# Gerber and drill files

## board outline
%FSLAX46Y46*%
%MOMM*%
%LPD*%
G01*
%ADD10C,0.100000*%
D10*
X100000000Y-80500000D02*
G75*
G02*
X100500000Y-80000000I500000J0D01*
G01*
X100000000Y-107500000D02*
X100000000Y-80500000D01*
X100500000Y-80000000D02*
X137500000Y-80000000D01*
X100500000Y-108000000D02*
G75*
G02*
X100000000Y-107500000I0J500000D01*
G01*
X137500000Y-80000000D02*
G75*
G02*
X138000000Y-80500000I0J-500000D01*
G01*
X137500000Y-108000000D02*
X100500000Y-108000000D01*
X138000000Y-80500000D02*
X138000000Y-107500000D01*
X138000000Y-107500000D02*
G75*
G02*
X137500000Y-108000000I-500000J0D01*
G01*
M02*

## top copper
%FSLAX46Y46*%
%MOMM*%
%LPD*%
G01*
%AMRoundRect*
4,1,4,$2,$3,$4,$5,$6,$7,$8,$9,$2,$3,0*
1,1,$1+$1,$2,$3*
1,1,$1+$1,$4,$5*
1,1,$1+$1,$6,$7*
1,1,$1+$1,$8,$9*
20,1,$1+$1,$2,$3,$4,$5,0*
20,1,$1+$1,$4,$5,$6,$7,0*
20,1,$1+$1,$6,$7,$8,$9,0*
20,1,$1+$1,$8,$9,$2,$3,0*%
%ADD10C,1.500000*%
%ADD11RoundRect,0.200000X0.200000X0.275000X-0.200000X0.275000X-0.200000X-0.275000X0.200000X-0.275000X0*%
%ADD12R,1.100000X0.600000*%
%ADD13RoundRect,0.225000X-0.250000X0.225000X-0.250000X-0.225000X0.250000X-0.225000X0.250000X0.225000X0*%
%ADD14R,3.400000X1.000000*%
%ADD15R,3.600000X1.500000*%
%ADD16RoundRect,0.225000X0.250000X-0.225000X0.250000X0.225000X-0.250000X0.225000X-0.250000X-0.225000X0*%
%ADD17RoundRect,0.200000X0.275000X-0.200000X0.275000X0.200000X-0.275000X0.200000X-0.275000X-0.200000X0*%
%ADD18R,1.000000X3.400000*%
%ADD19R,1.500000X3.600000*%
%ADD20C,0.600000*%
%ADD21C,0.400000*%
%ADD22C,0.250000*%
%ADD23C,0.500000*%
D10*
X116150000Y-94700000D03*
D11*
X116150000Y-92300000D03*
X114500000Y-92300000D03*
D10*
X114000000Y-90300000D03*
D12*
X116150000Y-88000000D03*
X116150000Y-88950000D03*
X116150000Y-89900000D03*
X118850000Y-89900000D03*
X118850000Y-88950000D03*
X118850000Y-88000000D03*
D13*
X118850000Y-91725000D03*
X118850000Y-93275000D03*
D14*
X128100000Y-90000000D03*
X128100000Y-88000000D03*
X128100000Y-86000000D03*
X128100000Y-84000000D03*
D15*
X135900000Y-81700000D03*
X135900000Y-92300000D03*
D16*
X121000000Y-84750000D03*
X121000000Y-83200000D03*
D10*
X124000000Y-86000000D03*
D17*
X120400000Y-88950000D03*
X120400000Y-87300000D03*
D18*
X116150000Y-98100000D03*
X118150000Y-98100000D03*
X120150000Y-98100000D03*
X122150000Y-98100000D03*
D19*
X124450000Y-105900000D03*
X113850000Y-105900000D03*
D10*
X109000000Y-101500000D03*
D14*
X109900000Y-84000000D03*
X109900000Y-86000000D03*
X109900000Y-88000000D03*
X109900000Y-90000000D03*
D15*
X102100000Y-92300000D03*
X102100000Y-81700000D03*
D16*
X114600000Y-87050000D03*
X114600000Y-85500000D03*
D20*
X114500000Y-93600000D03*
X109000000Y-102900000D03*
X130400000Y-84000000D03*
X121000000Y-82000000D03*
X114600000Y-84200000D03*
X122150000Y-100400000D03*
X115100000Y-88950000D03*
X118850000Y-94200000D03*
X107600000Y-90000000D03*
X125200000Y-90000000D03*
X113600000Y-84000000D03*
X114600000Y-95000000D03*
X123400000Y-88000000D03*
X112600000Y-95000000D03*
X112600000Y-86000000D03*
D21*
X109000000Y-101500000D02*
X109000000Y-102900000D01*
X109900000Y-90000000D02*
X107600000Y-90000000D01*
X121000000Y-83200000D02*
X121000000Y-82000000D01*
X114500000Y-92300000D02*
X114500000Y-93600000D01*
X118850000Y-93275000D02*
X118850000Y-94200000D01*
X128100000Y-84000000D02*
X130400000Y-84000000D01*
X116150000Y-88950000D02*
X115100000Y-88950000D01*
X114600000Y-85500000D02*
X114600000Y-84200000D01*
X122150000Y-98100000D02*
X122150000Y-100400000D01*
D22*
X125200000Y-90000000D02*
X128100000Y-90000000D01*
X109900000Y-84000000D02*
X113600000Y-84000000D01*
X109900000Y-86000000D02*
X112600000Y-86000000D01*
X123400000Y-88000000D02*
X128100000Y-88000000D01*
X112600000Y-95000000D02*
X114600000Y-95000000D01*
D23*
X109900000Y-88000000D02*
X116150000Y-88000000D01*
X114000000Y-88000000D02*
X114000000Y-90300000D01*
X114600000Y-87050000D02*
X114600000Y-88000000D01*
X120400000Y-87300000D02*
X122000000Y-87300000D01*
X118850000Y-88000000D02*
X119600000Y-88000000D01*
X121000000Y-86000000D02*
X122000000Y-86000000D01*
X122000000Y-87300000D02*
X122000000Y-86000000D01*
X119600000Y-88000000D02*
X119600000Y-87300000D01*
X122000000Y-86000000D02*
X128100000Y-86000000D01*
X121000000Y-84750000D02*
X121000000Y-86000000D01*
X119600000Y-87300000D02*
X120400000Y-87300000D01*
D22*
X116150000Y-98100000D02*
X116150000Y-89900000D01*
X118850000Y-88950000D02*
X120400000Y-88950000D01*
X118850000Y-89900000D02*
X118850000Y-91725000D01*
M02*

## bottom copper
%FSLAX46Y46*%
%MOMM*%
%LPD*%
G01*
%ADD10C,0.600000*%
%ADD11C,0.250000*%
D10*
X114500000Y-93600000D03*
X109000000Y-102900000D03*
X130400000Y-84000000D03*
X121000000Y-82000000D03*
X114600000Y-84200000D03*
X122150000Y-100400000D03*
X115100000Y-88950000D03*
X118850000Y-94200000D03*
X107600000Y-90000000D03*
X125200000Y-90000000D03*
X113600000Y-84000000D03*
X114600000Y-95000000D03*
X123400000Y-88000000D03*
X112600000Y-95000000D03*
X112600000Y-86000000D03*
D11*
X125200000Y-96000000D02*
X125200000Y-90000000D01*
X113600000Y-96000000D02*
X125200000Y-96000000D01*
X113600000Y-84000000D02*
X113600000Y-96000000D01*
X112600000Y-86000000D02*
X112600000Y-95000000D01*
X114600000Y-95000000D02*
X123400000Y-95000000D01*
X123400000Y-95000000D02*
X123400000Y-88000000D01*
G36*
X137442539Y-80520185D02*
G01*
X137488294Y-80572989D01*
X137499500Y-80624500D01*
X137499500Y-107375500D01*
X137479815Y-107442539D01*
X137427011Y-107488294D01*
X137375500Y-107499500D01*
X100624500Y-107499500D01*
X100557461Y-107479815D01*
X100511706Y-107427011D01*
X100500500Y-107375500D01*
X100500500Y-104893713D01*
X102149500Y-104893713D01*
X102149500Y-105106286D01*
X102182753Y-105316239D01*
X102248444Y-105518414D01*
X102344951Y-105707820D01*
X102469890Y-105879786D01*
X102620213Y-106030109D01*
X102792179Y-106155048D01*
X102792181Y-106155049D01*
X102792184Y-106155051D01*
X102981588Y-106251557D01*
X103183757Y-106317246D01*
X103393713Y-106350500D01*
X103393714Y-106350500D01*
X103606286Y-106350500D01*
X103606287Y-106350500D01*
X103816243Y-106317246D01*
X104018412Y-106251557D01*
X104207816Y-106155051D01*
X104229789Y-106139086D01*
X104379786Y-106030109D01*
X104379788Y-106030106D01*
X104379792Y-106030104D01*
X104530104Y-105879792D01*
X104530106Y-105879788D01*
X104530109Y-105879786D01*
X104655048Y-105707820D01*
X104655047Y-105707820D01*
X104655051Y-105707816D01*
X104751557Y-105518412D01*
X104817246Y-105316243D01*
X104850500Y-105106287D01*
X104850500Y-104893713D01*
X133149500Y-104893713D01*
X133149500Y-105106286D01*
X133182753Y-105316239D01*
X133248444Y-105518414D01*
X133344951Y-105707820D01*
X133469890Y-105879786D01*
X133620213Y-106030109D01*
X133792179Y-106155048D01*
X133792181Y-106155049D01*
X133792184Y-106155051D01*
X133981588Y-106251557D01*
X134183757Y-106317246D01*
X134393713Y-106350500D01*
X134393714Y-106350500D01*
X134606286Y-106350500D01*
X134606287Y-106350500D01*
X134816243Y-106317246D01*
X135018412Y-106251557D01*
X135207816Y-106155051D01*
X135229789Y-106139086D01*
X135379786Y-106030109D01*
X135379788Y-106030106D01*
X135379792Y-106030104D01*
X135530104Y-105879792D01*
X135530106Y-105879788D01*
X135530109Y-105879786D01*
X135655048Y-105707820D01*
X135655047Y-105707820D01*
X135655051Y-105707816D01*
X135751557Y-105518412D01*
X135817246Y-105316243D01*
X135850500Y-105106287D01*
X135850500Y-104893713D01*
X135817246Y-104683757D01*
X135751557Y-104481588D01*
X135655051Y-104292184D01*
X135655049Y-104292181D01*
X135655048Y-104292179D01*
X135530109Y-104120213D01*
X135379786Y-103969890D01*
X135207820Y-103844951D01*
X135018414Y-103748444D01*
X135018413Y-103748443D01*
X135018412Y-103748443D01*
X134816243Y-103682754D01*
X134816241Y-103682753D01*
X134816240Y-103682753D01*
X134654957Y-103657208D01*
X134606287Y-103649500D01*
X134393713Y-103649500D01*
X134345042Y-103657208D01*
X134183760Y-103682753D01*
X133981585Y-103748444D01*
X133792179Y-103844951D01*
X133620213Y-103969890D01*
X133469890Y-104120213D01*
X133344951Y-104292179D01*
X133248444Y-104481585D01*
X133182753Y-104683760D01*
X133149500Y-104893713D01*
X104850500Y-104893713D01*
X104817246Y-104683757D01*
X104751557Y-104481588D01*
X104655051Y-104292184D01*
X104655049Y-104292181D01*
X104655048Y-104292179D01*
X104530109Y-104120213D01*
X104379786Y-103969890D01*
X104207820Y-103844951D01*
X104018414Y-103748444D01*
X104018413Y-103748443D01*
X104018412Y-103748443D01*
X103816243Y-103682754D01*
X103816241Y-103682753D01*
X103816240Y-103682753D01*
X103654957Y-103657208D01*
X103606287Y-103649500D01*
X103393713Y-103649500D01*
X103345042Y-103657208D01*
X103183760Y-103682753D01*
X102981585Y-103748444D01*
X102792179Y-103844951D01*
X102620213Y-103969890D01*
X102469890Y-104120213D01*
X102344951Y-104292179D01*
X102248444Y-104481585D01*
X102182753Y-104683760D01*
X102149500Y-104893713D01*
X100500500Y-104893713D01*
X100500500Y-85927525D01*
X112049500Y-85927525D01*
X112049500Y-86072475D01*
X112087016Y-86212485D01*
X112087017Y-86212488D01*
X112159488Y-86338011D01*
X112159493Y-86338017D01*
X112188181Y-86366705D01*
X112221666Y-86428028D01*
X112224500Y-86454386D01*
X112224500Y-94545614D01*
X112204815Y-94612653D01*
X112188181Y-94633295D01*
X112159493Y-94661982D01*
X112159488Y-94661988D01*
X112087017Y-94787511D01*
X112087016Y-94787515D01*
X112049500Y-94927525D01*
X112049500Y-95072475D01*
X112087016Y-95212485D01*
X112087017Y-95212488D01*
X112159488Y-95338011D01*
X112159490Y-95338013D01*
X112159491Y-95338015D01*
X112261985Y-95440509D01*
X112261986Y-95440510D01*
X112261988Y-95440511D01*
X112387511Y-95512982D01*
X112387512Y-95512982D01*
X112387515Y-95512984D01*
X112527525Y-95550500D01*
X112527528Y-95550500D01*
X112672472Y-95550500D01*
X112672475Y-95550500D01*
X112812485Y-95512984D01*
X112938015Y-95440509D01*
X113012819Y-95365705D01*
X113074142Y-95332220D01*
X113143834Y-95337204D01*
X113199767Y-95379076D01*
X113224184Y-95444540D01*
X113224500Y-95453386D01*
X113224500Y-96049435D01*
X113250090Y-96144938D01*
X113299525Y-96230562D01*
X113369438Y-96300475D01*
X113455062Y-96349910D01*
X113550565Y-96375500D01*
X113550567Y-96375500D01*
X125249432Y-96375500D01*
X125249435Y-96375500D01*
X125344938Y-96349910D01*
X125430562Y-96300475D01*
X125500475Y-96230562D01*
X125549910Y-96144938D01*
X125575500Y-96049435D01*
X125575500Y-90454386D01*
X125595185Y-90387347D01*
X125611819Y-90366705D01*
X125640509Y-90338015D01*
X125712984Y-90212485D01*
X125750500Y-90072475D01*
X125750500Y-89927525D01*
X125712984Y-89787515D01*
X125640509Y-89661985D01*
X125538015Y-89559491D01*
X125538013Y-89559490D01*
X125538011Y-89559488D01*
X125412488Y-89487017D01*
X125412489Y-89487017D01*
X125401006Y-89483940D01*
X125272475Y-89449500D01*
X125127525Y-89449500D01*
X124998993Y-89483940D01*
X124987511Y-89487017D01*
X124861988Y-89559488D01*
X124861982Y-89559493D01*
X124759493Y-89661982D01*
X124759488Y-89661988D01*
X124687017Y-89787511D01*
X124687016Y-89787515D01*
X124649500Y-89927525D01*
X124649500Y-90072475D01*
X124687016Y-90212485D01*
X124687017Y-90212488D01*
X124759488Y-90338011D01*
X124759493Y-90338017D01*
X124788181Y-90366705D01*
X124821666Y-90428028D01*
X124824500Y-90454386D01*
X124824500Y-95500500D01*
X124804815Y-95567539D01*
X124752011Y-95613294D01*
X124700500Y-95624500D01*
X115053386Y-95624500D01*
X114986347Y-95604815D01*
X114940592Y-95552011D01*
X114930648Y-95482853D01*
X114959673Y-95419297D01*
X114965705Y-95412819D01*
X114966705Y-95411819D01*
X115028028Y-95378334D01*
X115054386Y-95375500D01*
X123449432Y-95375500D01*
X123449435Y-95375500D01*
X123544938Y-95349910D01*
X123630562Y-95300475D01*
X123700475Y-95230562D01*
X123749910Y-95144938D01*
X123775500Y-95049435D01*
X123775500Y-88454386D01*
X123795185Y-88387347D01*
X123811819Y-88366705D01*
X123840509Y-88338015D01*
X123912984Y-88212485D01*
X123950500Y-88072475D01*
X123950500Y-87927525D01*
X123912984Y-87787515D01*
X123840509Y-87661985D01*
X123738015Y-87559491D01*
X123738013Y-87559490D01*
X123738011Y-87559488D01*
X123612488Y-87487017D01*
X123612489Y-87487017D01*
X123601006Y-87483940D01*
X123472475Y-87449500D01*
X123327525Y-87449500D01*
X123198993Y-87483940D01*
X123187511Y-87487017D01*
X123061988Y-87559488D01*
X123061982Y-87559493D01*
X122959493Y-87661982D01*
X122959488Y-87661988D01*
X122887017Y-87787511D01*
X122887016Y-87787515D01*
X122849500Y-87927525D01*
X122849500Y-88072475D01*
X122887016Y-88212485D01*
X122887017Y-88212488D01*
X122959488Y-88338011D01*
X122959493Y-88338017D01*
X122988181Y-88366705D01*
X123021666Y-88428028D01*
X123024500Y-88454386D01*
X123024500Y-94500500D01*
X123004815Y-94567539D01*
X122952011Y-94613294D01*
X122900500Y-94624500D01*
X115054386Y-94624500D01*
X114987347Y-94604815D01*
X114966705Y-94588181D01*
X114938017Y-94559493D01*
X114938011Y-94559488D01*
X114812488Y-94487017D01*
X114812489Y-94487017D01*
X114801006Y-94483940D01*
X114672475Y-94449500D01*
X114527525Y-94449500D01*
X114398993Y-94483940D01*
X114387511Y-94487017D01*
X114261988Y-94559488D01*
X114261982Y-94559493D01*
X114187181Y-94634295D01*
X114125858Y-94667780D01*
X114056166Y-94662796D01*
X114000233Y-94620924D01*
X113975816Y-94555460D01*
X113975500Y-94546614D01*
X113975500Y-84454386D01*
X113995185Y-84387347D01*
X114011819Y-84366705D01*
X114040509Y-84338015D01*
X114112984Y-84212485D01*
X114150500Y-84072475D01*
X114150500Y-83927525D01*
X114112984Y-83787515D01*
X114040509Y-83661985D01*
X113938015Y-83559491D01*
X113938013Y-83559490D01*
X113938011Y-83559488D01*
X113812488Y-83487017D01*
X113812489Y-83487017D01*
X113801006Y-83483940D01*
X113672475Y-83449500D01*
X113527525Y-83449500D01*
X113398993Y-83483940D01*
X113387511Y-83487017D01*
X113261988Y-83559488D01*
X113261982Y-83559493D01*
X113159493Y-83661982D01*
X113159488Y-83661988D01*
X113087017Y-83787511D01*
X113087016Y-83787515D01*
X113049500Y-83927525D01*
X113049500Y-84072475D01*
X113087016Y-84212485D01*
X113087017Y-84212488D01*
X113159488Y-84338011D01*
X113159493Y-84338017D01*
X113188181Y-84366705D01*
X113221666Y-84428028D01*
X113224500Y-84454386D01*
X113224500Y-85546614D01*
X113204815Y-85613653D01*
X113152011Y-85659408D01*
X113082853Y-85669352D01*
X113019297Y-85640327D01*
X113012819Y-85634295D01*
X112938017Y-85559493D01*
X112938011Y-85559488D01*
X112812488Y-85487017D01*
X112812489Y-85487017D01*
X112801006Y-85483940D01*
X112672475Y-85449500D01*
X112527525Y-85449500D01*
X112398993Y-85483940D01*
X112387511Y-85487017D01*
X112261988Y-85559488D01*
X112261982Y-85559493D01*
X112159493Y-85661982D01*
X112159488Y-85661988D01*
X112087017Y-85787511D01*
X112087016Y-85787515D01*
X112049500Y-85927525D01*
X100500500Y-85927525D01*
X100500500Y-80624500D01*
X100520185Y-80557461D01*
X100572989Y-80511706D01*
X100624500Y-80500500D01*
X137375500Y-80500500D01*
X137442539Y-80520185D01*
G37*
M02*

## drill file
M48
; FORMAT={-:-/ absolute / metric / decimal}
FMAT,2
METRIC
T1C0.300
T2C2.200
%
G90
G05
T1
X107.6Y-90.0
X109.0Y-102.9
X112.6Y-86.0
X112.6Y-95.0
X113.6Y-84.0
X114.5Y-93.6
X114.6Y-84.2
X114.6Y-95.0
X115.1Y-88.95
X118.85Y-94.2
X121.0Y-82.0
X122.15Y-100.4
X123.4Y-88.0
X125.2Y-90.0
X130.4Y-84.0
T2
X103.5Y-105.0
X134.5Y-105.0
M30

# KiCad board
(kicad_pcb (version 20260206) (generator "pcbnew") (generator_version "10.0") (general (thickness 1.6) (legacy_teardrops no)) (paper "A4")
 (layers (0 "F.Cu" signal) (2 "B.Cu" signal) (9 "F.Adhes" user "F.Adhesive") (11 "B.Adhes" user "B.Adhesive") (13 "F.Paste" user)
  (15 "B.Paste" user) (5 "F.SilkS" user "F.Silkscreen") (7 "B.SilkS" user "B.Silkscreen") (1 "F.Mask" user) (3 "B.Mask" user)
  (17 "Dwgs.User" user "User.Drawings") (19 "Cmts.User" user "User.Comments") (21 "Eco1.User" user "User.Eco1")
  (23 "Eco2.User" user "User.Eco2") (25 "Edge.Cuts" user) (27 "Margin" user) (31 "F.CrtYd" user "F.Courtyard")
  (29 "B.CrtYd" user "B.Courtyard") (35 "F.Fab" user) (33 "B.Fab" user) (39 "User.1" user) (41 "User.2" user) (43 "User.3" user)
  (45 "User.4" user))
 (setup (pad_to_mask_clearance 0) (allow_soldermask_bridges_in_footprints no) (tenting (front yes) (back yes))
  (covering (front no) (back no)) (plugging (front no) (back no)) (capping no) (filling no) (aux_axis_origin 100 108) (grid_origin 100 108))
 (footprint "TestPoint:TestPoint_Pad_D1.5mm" (layer "F.Cu") (at 116.15 94.7)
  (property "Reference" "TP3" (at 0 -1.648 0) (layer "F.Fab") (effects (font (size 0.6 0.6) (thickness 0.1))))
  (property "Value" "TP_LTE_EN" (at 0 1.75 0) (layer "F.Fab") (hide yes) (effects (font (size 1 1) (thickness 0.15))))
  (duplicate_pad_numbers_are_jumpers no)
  (pad "1" smd circle (at 0 0) (size 1.5 1.5) (layers "F.Cu" "F.Mask") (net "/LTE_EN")))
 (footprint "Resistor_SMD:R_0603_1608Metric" (layer "F.Cu") (at 115.325 92.3 180)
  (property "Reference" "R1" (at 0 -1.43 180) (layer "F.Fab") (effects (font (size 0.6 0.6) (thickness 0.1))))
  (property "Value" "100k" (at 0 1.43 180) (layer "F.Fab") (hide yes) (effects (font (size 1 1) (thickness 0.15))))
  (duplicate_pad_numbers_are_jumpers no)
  (pad "1" smd roundrect (at -0.825 0 180) (size 0.8 0.95) (layers "F.Cu" "F.Mask" "F.Paste") (roundrect_rratio 0.25) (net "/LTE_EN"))
  (pad "2" smd roundrect (at 0.825 0 180) (size 0.8 0.95) (layers "F.Cu" "F.Mask" "F.Paste") (roundrect_rratio 0.25) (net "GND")))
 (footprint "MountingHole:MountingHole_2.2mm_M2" (layer "F.Cu") (at 134.5 105)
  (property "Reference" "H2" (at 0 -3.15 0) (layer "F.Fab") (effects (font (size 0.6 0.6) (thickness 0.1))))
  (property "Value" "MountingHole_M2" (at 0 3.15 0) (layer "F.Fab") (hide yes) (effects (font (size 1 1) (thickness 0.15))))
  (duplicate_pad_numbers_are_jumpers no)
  (pad "" np_thru_hole circle (at 0 0) (size 2.2 2.2) (drill 2.2) (layers "*.Cu" "*.Mask")))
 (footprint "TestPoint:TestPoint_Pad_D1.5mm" (layer "F.Cu") (at 114 90.3)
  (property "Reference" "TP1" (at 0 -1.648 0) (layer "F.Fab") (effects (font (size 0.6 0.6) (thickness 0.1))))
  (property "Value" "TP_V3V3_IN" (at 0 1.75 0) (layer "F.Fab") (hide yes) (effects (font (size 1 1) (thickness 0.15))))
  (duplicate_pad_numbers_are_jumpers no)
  (pad "1" smd circle (at 0 0) (size 1.5 1.5) (layers "F.Cu" "F.Mask") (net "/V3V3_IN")))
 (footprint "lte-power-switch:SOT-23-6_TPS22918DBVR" (layer "F.Cu") (at 117.5 88.95 180)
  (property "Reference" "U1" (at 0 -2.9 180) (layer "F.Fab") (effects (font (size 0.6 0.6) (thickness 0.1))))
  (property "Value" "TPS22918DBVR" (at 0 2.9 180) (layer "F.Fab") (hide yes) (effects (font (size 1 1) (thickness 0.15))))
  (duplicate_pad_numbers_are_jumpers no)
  (pad "1" smd rect (at 1.35 0.95 180) (size 1.1 0.6) (layers "F.Cu" "F.Mask" "F.Paste") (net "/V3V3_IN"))
  (pad "2" smd rect (at 1.35 0 180) (size 1.1 0.6) (layers "F.Cu" "F.Mask" "F.Paste") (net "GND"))
  (pad "3" smd rect (at 1.35 -0.95 180) (size 1.1 0.6) (layers "F.Cu" "F.Mask" "F.Paste") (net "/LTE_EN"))
  (pad "4" smd rect (at -1.35 -0.95 180) (size 1.1 0.6) (layers "F.Cu" "F.Mask" "F.Paste") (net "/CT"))
  (pad "5" smd rect (at -1.35 0 180) (size 1.1 0.6) (layers "F.Cu" "F.Mask" "F.Paste") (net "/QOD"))
  (pad "6" smd rect (at -1.35 0.95 180) (size 1.1 0.6) (layers "F.Cu" "F.Mask" "F.Paste") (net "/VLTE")))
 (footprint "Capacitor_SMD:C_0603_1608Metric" (layer "F.Cu") (at 118.85 92.5 -90)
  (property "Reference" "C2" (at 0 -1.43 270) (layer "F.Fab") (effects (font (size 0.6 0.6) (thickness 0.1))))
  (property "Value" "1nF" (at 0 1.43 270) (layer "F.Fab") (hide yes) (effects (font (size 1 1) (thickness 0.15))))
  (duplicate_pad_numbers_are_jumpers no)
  (pad "1" smd roundrect (at -0.775 0 270) (size 0.9 0.95) (layers "F.Cu" "F.Mask" "F.Paste") (roundrect_rratio 0.25) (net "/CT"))
  (pad "2" smd roundrect (at 0.775 0 270) (size 0.9 0.95) (layers "F.Cu" "F.Mask" "F.Paste") (roundrect_rratio 0.25) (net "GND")))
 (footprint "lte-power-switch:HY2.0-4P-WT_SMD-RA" (layer "F.Cu") (at 132 87 90)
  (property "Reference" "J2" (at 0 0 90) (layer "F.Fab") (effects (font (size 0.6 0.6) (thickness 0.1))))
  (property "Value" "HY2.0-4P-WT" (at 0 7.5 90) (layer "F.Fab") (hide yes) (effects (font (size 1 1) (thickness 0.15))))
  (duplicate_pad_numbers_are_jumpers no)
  (pad "1" smd rect (at -3 -3.9 90) (size 1 3.4) (layers "F.Cu" "F.Mask" "F.Paste") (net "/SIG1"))
  (pad "2" smd rect (at -1 -3.9 90) (size 1 3.4) (layers "F.Cu" "F.Mask" "F.Paste") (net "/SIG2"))
  (pad "3" smd rect (at 1 -3.9 90) (size 1 3.4) (layers "F.Cu" "F.Mask" "F.Paste") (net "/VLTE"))
  (pad "4" smd rect (at 3 -3.9 90) (size 1 3.4) (layers "F.Cu" "F.Mask" "F.Paste") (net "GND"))
  (pad "5" smd rect (at 5.3 3.9 90) (size 1.5 3.6) (layers "F.Cu" "F.Mask" "F.Paste"))
  (pad "6" smd rect (at -5.3 3.9 90) (size 1.5 3.6) (layers "F.Cu" "F.Mask" "F.Paste")))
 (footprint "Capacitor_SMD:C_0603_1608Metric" (layer "F.Cu") (at 121 83.975 90)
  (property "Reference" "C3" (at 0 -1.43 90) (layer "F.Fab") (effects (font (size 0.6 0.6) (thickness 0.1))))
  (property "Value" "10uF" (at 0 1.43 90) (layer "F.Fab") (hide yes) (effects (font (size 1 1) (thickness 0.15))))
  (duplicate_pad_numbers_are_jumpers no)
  (pad "1" smd roundrect (at -0.775 0 90) (size 0.9 0.95) (layers "F.Cu" "F.Mask" "F.Paste") (roundrect_rratio 0.25) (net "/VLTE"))
  (pad "2" smd roundrect (at 0.775 0 90) (size 0.9 0.95) (layers "F.Cu" "F.Mask" "F.Paste") (roundrect_rratio 0.25) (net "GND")))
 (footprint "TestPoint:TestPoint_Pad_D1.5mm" (layer "F.Cu") (at 124 86)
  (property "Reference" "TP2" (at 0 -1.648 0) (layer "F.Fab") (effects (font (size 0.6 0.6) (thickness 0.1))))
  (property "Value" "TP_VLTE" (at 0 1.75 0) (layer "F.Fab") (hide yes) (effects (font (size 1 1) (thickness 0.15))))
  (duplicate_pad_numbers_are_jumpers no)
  (pad "1" smd circle (at 0 0) (size 1.5 1.5) (layers "F.Cu" "F.Mask") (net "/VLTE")))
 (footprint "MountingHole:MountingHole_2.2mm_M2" (layer "F.Cu") (at 103.5 105)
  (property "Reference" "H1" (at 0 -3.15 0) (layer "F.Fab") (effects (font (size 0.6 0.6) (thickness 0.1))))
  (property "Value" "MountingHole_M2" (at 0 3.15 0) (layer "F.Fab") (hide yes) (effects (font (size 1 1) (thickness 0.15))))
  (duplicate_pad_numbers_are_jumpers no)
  (pad "" np_thru_hole circle (at 0 0) (size 2.2 2.2) (drill 2.2) (layers "*.Cu" "*.Mask")))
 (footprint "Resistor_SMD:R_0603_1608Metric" (layer "F.Cu") (at 120.4 88.125 90)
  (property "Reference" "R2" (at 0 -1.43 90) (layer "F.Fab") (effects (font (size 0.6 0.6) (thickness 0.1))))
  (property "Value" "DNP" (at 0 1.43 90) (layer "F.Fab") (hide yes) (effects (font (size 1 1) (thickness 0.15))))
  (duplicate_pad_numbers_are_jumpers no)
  (pad "1" smd roundrect (at -0.825 0 90) (size 0.8 0.95) (layers "F.Cu" "F.Mask" "F.Paste") (roundrect_rratio 0.25) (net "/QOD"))
  (pad "2" smd roundrect (at 0.825 0 90) (size 0.8 0.95) (layers "F.Cu" "F.Mask" "F.Paste") (roundrect_rratio 0.25) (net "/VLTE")))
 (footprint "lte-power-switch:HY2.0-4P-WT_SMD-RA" (layer "F.Cu") (at 119.15 102)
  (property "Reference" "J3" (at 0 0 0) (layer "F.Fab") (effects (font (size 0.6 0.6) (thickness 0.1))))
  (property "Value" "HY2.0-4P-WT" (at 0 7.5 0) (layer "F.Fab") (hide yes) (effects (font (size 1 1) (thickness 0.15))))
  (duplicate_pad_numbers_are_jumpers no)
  (pad "1" smd rect (at -3 -3.9) (size 1 3.4) (layers "F.Cu" "F.Mask" "F.Paste") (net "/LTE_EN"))
  (pad "2" smd rect (at -1 -3.9) (size 1 3.4) (layers "F.Cu" "F.Mask" "F.Paste") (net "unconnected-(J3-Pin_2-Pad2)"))
  (pad "3" smd rect (at 1 -3.9) (size 1 3.4) (layers "F.Cu" "F.Mask" "F.Paste") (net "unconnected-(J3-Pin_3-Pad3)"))
  (pad "4" smd rect (at 3 -3.9) (size 1 3.4) (layers "F.Cu" "F.Mask" "F.Paste") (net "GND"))
  (pad "5" smd rect (at 5.3 3.9) (size 1.5 3.6) (layers "F.Cu" "F.Mask" "F.Paste"))
  (pad "6" smd rect (at -5.3 3.9) (size 1.5 3.6) (layers "F.Cu" "F.Mask" "F.Paste")))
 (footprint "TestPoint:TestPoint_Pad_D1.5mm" (layer "F.Cu") (at 109 101.5)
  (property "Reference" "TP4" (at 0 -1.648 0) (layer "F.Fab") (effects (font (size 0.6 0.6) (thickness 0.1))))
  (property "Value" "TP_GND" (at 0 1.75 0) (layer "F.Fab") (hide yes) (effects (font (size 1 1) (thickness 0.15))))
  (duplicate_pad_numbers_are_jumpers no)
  (pad "1" smd circle (at 0 0) (size 1.5 1.5) (layers "F.Cu" "F.Mask") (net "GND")))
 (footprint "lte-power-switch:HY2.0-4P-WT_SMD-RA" (layer "F.Cu") (at 106 87 -90)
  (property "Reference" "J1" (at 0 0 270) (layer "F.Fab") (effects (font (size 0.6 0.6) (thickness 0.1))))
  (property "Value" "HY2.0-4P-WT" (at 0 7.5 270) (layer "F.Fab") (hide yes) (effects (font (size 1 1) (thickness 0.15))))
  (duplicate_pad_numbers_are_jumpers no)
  (pad "1" smd rect (at -3 -3.9 270) (size 1 3.4) (layers "F.Cu" "F.Mask" "F.Paste") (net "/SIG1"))
  (pad "2" smd rect (at -1 -3.9 270) (size 1 3.4) (layers "F.Cu" "F.Mask" "F.Paste") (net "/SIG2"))
  (pad "3" smd rect (at 1 -3.9 270) (size 1 3.4) (layers "F.Cu" "F.Mask" "F.Paste") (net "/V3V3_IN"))
  (pad "4" smd rect (at 3 -3.9 270) (size 1 3.4) (layers "F.Cu" "F.Mask" "F.Paste") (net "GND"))
  (pad "5" smd rect (at 5.3 3.9 270) (size 1.5 3.6) (layers "F.Cu" "F.Mask" "F.Paste"))
  (pad "6" smd rect (at -5.3 3.9 270) (size 1.5 3.6) (layers "F.Cu" "F.Mask" "F.Paste")))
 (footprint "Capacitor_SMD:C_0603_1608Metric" (layer "F.Cu") (at 114.6 86.275 90)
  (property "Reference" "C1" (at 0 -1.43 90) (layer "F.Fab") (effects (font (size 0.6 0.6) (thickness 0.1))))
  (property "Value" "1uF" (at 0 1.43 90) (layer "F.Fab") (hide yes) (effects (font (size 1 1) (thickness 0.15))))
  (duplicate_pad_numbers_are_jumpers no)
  (pad "1" smd roundrect (at -0.775 0 90) (size 0.9 0.95) (layers "F.Cu" "F.Mask" "F.Paste") (roundrect_rratio 0.25) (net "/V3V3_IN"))
  (pad "2" smd roundrect (at 0.775 0 90) (size 0.9 0.95) (layers "F.Cu" "F.Mask" "F.Paste") (roundrect_rratio 0.25) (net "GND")))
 (gr_arc (start 100 80.5) (mid 100.146446 80.146446) (end 100.5 80) (stroke (width 0.1) (type default)) (layer "Edge.Cuts"))
 (gr_line (start 100 107.5) (end 100 80.5) (stroke (width 0.1) (type default)) (layer "Edge.Cuts"))
 (gr_line (start 100.5 80) (end 137.5 80) (stroke (width 0.1) (type default)) (layer "Edge.Cuts"))
 (gr_arc (start 100.5 108) (mid 100.146446 107.853553) (end 100 107.5) (stroke (width 0.1) (type default)) (layer "Edge.Cuts"))
 (gr_arc (start 137.5 80) (mid 137.853553 80.146446) (end 138 80.5) (stroke (width 0.1) (type default)) (layer "Edge.Cuts"))
 (gr_line (start 137.5 108) (end 100.5 108) (stroke (width 0.1) (type default)) (layer "Edge.Cuts"))
 (gr_line (start 138 80.5) (end 138 107.5) (stroke (width 0.1) (type default)) (layer "Edge.Cuts"))
 (gr_arc (start 138 107.5) (mid 137.853553 107.853553) (end 137.5 108) (stroke (width 0.1) (type default)) (layer "Edge.Cuts"))
 (segment (start 109 101.5) (end 109 102.9) (width 0.4) (layer "F.Cu") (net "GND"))
 (segment (start 109.9 90) (end 107.6 90) (width 0.4) (layer "F.Cu") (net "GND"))
 (segment (start 121 83.2) (end 121 82) (width 0.4) (layer "F.Cu") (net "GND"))
 (segment (start 114.5 92.3) (end 114.5 93.6) (width 0.4) (layer "F.Cu") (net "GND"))
 (segment (start 118.85 93.275) (end 118.85 94.2) (width 0.4) (layer "F.Cu") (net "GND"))
 (segment (start 128.1 84) (end 130.4 84) (width 0.4) (layer "F.Cu") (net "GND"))
 (segment (start 116.15 88.95) (end 115.1 88.95) (width 0.4) (layer "F.Cu") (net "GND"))
 (segment (start 114.6 85.5) (end 114.6 84.2) (width 0.4) (layer "F.Cu") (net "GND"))
 (segment (start 122.15 98.1) (end 122.15 100.4) (width 0.4) (layer "F.Cu") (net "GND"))
 (via (at 114.5 93.6) (size 0.6) (drill 0.3) (layers "F.Cu" "B.Cu") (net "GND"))
 (via (at 109 102.9) (size 0.6) (drill 0.3) (layers "F.Cu" "B.Cu") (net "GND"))
 (via (at 130.4 84) (size 0.6) (drill 0.3) (layers "F.Cu" "B.Cu") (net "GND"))
 (via (at 121 82) (size 0.6) (drill 0.3) (layers "F.Cu" "B.Cu") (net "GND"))
 (via (at 114.6 84.2) (size 0.6) (drill 0.3) (layers "F.Cu" "B.Cu") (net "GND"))
 (via (at 122.15 100.4) (size 0.6) (drill 0.3) (layers "F.Cu" "B.Cu") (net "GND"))
 (via (at 115.1 88.95) (size 0.6) (drill 0.3) (layers "F.Cu" "B.Cu") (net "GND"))
 (via (at 118.85 94.2) (size 0.6) (drill 0.3) (layers "F.Cu" "B.Cu") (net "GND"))
 (via (at 107.6 90) (size 0.6) (drill 0.3) (layers "F.Cu" "B.Cu") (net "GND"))
 (segment (start 125.2 90) (end 128.1 90) (width 0.25) (layer "F.Cu") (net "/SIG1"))
 (segment (start 109.9 84) (end 113.6 84) (width 0.25) (layer "F.Cu") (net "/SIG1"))
 (via (at 125.2 90) (size 0.6) (drill 0.3) (layers "F.Cu" "B.Cu") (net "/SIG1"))
 (via (at 113.6 84) (size 0.6) (drill 0.3) (layers "F.Cu" "B.Cu") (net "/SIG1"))
 (segment (start 125.2 96) (end 125.2 90) (width 0.25) (layer "B.Cu") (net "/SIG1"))
 (segment (start 113.6 96) (end 125.2 96) (width 0.25) (layer "B.Cu") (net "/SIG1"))
 (segment (start 113.6 84) (end 113.6 96) (width 0.25) (layer "B.Cu") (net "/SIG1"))
 (segment (start 109.9 86) (end 112.6 86) (width 0.25) (layer "F.Cu") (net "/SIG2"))
 (segment (start 123.4 88) (end 128.1 88) (width 0.25) (layer "F.Cu") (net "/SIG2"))
 (segment (start 112.6 95) (end 114.6 95) (width 0.25) (layer "F.Cu") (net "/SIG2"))
 (via (at 114.6 95) (size 0.6) (drill 0.3) (layers "F.Cu" "B.Cu") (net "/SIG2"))
 (via (at 123.4 88) (size 0.6) (drill 0.3) (layers "F.Cu" "B.Cu") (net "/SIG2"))
 (via (at 112.6 95) (size 0.6) (drill 0.3) (layers "F.Cu" "B.Cu") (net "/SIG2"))
 (via (at 112.6 86) (size 0.6) (drill 0.3) (layers "F.Cu" "B.Cu") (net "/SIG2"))
 (segment (start 112.6 86) (end 112.6 95) (width 0.25) (layer "B.Cu") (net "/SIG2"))
 (segment (start 114.6 95) (end 123.4 95) (width 0.25) (layer "B.Cu") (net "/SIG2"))
 (segment (start 123.4 95) (end 123.4 88) (width 0.25) (layer "B.Cu") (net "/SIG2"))
 (segment (start 109.9 88) (end 116.15 88) (width 0.5) (layer "F.Cu") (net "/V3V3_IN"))
 (segment (start 114 88) (end 114 90.3) (width 0.5) (layer "F.Cu") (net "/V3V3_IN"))
 (segment (start 114.6 87.05) (end 114.6 88) (width 0.5) (layer "F.Cu") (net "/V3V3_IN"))
 (segment (start 120.4 87.3) (end 122 87.3) (width 0.5) (layer "F.Cu") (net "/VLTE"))
 (segment (start 118.85 88) (end 119.6 88) (width 0.5) (layer "F.Cu") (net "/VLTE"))
 (segment (start 121 86) (end 122 86) (width 0.5) (layer "F.Cu") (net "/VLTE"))
 (segment (start 122 87.3) (end 122 86) (width 0.5) (layer "F.Cu") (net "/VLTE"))
 (segment (start 119.6 88) (end 119.6 87.3) (width 0.5) (layer "F.Cu") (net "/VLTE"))
 (segment (start 122 86) (end 128.1 86) (width 0.5) (layer "F.Cu") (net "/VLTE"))
 (segment (start 121 84.75) (end 121 86) (width 0.5) (layer "F.Cu") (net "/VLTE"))
 (segment (start 119.6 87.3) (end 120.4 87.3) (width 0.5) (layer "F.Cu") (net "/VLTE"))
 (segment (start 116.15 98.1) (end 116.15 89.9) (width 0.25) (layer "F.Cu") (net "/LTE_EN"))
 (segment (start 118.85 88.95) (end 120.4 88.95) (width 0.25) (layer "F.Cu") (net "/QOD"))
 (segment (start 118.85 89.9) (end 118.85 91.725) (width 0.25) (layer "F.Cu") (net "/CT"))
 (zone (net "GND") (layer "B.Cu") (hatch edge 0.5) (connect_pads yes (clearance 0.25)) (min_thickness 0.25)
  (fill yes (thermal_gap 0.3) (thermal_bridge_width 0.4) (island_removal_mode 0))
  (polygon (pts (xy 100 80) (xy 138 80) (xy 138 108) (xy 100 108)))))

